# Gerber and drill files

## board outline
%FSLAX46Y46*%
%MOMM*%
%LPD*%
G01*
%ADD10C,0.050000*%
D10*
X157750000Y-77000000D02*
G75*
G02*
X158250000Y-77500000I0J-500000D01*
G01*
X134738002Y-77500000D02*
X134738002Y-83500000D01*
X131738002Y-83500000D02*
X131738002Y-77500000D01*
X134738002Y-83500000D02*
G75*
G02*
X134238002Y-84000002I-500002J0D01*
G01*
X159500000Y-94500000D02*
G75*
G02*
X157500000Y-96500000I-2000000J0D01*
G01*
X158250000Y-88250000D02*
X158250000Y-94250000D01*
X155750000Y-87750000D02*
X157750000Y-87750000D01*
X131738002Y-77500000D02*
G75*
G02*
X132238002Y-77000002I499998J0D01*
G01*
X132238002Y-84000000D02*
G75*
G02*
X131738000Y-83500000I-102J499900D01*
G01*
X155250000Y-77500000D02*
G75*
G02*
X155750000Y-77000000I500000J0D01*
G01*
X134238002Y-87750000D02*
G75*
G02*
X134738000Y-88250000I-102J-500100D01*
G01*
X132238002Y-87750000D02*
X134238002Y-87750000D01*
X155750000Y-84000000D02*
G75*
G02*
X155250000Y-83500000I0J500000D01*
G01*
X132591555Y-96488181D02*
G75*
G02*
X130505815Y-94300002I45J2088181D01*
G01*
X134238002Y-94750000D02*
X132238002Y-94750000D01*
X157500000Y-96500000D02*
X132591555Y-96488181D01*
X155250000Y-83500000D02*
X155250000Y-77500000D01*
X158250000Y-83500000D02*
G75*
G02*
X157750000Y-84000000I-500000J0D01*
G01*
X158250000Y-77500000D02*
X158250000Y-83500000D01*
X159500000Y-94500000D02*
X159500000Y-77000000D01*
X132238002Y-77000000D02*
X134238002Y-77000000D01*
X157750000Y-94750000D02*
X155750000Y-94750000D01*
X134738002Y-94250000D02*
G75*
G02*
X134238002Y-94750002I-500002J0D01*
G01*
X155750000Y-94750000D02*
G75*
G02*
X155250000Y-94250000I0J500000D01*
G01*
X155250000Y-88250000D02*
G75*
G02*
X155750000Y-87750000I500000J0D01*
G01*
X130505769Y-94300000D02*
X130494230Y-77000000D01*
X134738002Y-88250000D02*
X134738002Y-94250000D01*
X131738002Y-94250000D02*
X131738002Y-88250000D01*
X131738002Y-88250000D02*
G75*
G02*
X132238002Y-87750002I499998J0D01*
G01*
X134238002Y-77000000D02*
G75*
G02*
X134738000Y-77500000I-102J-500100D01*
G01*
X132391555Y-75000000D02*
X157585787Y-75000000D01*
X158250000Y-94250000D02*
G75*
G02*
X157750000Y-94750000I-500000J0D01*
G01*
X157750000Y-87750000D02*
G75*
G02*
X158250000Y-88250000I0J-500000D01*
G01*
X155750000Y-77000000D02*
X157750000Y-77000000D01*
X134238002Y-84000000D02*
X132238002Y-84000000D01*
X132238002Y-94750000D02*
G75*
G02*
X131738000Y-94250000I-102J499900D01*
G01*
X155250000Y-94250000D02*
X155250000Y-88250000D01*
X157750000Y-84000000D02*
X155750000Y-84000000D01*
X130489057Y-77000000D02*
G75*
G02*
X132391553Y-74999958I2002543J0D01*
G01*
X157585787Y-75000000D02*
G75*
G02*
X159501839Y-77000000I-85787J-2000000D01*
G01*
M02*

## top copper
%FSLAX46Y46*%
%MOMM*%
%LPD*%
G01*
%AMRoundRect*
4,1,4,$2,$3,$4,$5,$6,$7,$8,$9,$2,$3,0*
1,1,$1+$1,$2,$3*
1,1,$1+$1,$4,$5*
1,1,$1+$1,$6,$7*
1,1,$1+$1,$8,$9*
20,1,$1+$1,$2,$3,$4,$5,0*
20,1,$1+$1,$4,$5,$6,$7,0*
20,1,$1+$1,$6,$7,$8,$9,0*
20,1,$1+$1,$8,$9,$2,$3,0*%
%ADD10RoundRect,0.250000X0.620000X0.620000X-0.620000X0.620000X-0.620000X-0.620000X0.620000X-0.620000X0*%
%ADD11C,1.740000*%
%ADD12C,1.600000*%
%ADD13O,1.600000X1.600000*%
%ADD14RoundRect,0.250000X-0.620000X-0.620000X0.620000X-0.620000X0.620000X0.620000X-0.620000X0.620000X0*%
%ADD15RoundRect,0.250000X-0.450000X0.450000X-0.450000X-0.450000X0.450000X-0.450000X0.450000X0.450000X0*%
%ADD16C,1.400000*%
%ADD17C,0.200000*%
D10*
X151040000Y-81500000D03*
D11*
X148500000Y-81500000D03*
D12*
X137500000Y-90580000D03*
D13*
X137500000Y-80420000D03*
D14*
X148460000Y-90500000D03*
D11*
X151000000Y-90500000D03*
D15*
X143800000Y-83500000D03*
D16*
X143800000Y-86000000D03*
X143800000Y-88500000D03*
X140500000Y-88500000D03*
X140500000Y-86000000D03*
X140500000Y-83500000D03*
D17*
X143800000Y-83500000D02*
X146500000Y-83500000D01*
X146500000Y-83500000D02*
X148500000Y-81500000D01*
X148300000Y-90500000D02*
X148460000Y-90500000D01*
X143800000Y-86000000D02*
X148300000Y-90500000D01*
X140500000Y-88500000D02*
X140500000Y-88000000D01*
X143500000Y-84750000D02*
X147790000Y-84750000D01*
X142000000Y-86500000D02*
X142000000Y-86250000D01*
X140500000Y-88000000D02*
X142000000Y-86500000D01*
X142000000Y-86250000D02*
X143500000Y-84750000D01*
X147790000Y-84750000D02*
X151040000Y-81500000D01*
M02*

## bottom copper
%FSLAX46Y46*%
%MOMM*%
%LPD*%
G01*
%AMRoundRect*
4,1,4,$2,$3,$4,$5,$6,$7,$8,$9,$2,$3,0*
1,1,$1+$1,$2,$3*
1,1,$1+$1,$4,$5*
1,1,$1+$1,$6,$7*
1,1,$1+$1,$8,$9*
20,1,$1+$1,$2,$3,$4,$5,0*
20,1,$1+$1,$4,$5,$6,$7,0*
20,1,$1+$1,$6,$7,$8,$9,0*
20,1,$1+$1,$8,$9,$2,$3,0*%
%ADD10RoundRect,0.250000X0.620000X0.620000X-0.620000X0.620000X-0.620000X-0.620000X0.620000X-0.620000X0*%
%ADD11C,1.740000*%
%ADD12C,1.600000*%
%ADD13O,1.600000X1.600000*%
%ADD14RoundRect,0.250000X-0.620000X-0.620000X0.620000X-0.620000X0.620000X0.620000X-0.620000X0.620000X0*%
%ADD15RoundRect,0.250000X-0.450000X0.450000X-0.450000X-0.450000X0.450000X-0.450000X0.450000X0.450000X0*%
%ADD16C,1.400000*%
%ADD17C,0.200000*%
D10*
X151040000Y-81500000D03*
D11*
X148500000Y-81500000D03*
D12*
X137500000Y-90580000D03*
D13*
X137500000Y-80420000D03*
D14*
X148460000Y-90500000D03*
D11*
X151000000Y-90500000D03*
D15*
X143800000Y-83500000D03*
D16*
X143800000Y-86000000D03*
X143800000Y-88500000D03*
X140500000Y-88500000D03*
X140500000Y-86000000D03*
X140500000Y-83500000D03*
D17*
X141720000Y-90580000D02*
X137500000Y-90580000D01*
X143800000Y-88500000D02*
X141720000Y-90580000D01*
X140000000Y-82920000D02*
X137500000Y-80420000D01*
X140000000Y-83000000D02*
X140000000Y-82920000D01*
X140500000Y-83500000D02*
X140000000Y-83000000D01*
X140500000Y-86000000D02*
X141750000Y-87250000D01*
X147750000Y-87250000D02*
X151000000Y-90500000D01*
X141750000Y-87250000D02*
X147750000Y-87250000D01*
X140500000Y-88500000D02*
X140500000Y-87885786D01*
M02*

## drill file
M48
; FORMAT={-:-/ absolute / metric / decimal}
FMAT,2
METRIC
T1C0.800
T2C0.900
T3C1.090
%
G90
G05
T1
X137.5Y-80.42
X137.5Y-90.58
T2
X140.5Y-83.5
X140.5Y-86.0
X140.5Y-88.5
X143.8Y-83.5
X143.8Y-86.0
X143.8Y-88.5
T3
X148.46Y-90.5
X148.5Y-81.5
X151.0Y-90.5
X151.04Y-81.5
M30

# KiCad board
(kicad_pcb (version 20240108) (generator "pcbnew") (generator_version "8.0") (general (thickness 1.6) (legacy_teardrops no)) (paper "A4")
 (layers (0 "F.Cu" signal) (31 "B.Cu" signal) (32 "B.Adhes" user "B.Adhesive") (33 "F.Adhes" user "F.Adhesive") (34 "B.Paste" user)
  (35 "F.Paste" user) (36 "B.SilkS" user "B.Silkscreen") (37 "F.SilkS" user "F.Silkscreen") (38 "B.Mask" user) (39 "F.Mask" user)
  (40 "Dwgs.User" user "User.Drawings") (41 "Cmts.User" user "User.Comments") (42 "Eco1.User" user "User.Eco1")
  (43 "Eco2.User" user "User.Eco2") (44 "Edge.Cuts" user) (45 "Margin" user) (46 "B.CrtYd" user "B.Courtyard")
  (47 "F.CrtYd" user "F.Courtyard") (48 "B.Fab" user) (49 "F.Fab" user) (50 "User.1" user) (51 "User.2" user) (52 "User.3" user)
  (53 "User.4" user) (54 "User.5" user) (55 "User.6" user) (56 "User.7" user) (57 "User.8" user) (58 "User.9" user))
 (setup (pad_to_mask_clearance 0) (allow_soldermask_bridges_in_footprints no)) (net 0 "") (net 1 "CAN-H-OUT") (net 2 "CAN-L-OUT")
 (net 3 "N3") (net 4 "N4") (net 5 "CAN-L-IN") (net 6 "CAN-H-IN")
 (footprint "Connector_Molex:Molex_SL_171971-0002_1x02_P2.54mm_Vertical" (layer "F.Cu") (at 151.04 81.5 180)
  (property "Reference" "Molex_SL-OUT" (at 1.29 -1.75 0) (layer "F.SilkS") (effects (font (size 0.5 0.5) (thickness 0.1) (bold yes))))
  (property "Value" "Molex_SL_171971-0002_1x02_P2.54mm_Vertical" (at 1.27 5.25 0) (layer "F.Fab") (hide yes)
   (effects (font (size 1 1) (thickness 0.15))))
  (pad "1" thru_hole roundrect (at 0 0 180) (size 1.74 1.74) (drill 1.09) (layers "*.Cu" "*.Mask") (remove_unused_layers no)
   (roundrect_rratio 0.143678) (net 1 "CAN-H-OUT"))
  (pad "2" thru_hole circle (at 2.54 0 180) (size 1.74 1.74) (drill 1.09) (layers "*.Cu" "*.Mask") (remove_unused_layers no)
   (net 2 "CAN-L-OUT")))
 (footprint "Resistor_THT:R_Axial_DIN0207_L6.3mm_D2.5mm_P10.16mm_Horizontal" (layer "F.Cu") (at 137.5 90.58 90)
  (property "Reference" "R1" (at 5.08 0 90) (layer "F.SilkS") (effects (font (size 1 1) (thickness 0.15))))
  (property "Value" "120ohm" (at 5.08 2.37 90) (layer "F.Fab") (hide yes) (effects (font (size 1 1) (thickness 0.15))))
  (pad "1" thru_hole circle (at 0 0 90) (size 1.6 1.6) (drill 0.8) (layers "*.Cu" "*.Mask") (remove_unused_layers no) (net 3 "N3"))
  (pad "2" thru_hole oval (at 10.16 0 90) (size 1.6 1.6) (drill 0.8) (layers "*.Cu" "*.Mask") (remove_unused_layers no) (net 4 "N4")))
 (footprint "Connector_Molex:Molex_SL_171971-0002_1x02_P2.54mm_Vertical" (layer "F.Cu") (at 148.46 90.5)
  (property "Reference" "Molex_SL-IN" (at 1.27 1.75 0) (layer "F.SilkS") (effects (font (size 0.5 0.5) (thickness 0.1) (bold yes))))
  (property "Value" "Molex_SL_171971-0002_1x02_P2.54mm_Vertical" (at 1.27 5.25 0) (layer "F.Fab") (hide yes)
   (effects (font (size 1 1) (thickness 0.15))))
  (pad "1" thru_hole roundrect (at 0 0) (size 1.74 1.74) (drill 1.09) (layers "*.Cu" "*.Mask") (remove_unused_layers no)
   (roundrect_rratio 0.143678) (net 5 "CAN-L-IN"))
  (pad "2" thru_hole circle (at 2.54 0) (size 1.74 1.74) (drill 1.09) (layers "*.Cu" "*.Mask") (remove_unused_layers no) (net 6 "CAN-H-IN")))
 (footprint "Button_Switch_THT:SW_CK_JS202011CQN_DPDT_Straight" (layer "F.Cu") (at 143.8 83.5 -90)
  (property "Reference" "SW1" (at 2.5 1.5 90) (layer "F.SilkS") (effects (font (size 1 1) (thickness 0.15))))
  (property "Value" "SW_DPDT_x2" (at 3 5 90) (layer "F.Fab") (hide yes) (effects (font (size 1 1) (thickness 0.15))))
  (pad "1" thru_hole roundrect (at 0 0 270) (size 1.4 1.4) (drill 0.9) (layers "*.Cu" "*.Mask") (remove_unused_layers no)
   (roundrect_rratio 0.1785714286) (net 2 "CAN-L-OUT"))
  (pad "2" thru_hole circle (at 2.5 0 270) (size 1.4 1.4) (drill 0.9) (layers "*.Cu" "*.Mask") (remove_unused_layers no) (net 5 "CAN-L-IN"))
  (pad "3" thru_hole circle (at 5 0 270) (size 1.4 1.4) (drill 0.9) (layers "*.Cu" "*.Mask") (remove_unused_layers no) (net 3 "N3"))
  (pad "4" thru_hole circle (at 5 3.3 270) (size 1.4 1.4) (drill 0.9) (layers "*.Cu" "*.Mask") (remove_unused_layers no) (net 1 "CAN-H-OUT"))
  (pad "5" thru_hole circle (at 2.5 3.3 270) (size 1.4 1.4) (drill 0.9) (layers "*.Cu" "*.Mask") (remove_unused_layers no)
   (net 6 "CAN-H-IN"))
  (pad "6" thru_hole circle (at 0 3.3 270) (size 1.4 1.4) (drill 0.9) (layers "*.Cu" "*.Mask") (remove_unused_layers no) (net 4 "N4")))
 (gr_arc (start 157.75 77) (mid 158.103553 77.146447) (end 158.25 77.5) (stroke (width 0.05) (type default)) (layer "Edge.Cuts"))
 (gr_line (start 134.738002 77.5) (end 134.738002 83.5) (stroke (width 0.05) (type default)) (layer "Edge.Cuts"))
 (gr_line (start 131.738002 83.5) (end 131.738002 77.5) (stroke (width 0.05) (type default)) (layer "Edge.Cuts"))
 (gr_arc (start 134.738002 83.5) (mid 134.591558 83.85357) (end 134.238002 84) (stroke (width 0.05) (type default)) (layer "Edge.Cuts"))
 (gr_arc (start 159.5 94.5) (mid 158.914214 95.914214) (end 157.5 96.5) (stroke (width 0.05) (type default)) (layer "Edge.Cuts"))
 (gr_line (start 158.25 88.25) (end 158.25 94.25) (stroke (width 0.05) (type default)) (layer "Edge.Cuts"))
 (gr_line (start 155.75 87.75) (end 157.75 87.75) (stroke (width 0.05) (type default)) (layer "Edge.Cuts"))
 (gr_arc (start 131.738002 77.5) (mid 131.884451 77.146463) (end 132.238002 77) (stroke (width 0.05) (type default)) (layer "Edge.Cuts"))
 (gr_arc (start 132.238002 84) (mid 131.884418 83.85357) (end 131.738002 83.5) (stroke (width 0.05) (type default)) (layer "Edge.Cuts"))
 (gr_arc (start 155.25 77.5) (mid 155.396447 77.146447) (end 155.75 77) (stroke (width 0.05) (type default)) (layer "Edge.Cuts"))
 (gr_arc (start 134.238002 87.75) (mid 134.591525 87.896463) (end 134.738002 88.25) (stroke (width 0.05) (type default)) (layer "Edge.Cuts"))
 (gr_line (start 132.238002 87.75) (end 134.238002 87.75) (stroke (width 0.05) (type default)) (layer "Edge.Cuts"))
 (gr_arc (start 155.75 84) (mid 155.396447 83.853553) (end 155.25 83.5) (stroke (width 0.05) (type default)) (layer "Edge.Cuts"))
 (gr_arc (start 132.591555 96.488181) (mid 131.080046 95.840778) (end 130.50577 94.3) (stroke (width 0.05) (type default))
  (layer "Edge.Cuts"))
 (gr_line (start 134.238002 94.75) (end 132.238002 94.75) (stroke (width 0.05) (type default)) (layer "Edge.Cuts"))
 (gr_line (start 157.5 96.5) (end 132.591555 96.488181) (stroke (width 0.05) (type default)) (layer "Edge.Cuts"))
 (gr_line (start 155.25 83.5) (end 155.25 77.5) (stroke (width 0.05) (type default)) (layer "Edge.Cuts"))
 (gr_arc (start 158.25 83.5) (mid 158.103553 83.853553) (end 157.75 84) (stroke (width 0.05) (type default)) (layer "Edge.Cuts"))
 (gr_line (start 158.25 77.5) (end 158.25 83.5) (stroke (width 0.05) (type default)) (layer "Edge.Cuts"))
 (gr_line (start 159.5 94.5) (end 159.5 77) (stroke (width 0.05) (type default)) (layer "Edge.Cuts"))
 (gr_line (start 132.238002 77) (end 134.238002 77) (stroke (width 0.05) (type default)) (layer "Edge.Cuts"))
 (gr_line (start 157.75 94.75) (end 155.75 94.75) (stroke (width 0.05) (type default)) (layer "Edge.Cuts"))
 (gr_arc (start 134.738002 94.25) (mid 134.591558 94.60357) (end 134.238002 94.75) (stroke (width 0.05) (type default)) (layer "Edge.Cuts"))
 (gr_arc (start 155.75 94.75) (mid 155.396447 94.603553) (end 155.25 94.25) (stroke (width 0.05) (type default)) (layer "Edge.Cuts"))
 (gr_arc (start 155.25 88.25) (mid 155.396447 87.896447) (end 155.75 87.75) (stroke (width 0.05) (type default)) (layer "Edge.Cuts"))
 (gr_line (start 130.505769 94.3) (end 130.49423 77) (stroke (width 0.05) (type default)) (layer "Edge.Cuts"))
 (gr_line (start 134.738002 88.25) (end 134.738002 94.25) (stroke (width 0.05) (type default)) (layer "Edge.Cuts"))
 (gr_line (start 131.738002 94.25) (end 131.738002 88.25) (stroke (width 0.05) (type default)) (layer "Edge.Cuts"))
 (gr_arc (start 131.738002 88.25) (mid 131.884451 87.896463) (end 132.238002 87.75) (stroke (width 0.05) (type default)) (layer "Edge.Cuts"))
 (gr_arc (start 134.238002 77) (mid 134.591525 77.146463) (end 134.738002 77.5) (stroke (width 0.05) (type default)) (layer "Edge.Cuts"))
 (gr_line (start 132.391555 75) (end 157.585787 75) (stroke (width 0.05) (type default)) (layer "Edge.Cuts"))
 (gr_arc (start 158.25 94.25) (mid 158.103553 94.603553) (end 157.75 94.75) (stroke (width 0.05) (type default)) (layer "Edge.Cuts"))
 (gr_arc (start 157.75 87.75) (mid 158.103553 87.896447) (end 158.25 88.25) (stroke (width 0.05) (type default)) (layer "Edge.Cuts"))
 (gr_line (start 155.75 77) (end 157.75 77) (stroke (width 0.05) (type default)) (layer "Edge.Cuts"))
 (gr_line (start 134.238002 84) (end 132.238002 84) (stroke (width 0.05) (type default)) (layer "Edge.Cuts"))
 (gr_arc (start 132.238002 94.75) (mid 131.884418 94.60357) (end 131.738002 94.25) (stroke (width 0.05) (type default)) (layer "Edge.Cuts"))
 (gr_line (start 155.25 94.25) (end 155.25 88.25) (stroke (width 0.05) (type default)) (layer "Edge.Cuts"))
 (gr_line (start 157.75 84) (end 155.75 84) (stroke (width 0.05) (type default)) (layer "Edge.Cuts"))
 (gr_arc (start 130.489057 77) (mid 131.04065 75.619828) (end 132.391555 75) (stroke (width 0.05) (type default)) (layer "Edge.Cuts"))
 (gr_arc (start 157.585787 75) (mid 158.945526 75.615148) (end 159.501839 77) (stroke (width 0.05) (type default)) (layer "Edge.Cuts"))
 (segment (start 141.72 90.58) (end 137.5 90.58) (width 0.2) (layer "B.Cu") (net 3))
 (segment (start 143.8 88.5) (end 141.72 90.58) (width 0.2) (layer "B.Cu") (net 3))
 (segment (start 140 82.92) (end 137.5 80.42) (width 0.2) (layer "B.Cu") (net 4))
 (segment (start 140 83) (end 140 82.92) (width 0.2) (layer "B.Cu") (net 4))
 (segment (start 140.5 83.5) (end 140 83) (width 0.2) (layer "B.Cu") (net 4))
 (segment (start 143.8 83.5) (end 146.5 83.5) (width 0.2) (layer "F.Cu") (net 2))
 (segment (start 146.5 83.5) (end 148.5 81.5) (width 0.2) (layer "F.Cu") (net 2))
 (segment (start 148.3 90.5) (end 148.46 90.5) (width 0.2) (layer "F.Cu") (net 5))
 (segment (start 143.8 86) (end 148.3 90.5) (width 0.2) (layer "F.Cu") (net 5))
 (segment (start 140.5 86) (end 141.75 87.25) (width 0.2) (layer "B.Cu") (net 6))
 (segment (start 147.75 87.25) (end 151 90.5) (width 0.2) (layer "B.Cu") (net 6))
 (segment (start 141.75 87.25) (end 147.75 87.25) (width 0.2) (layer "B.Cu") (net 6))
 (segment (start 140.5 88.5) (end 140.5 88) (width 0.2) (layer "F.Cu") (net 1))
 (segment (start 143.5 84.75) (end 147.79 84.75) (width 0.2) (layer "F.Cu") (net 1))
 (segment (start 142 86.5) (end 142 86.25) (width 0.2) (layer "F.Cu") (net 1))
 (segment (start 140.5 88) (end 142 86.5) (width 0.2) (layer "F.Cu") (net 1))
 (segment (start 142 86.25) (end 143.5 84.75) (width 0.2) (layer "F.Cu") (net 1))
 (segment (start 147.79 84.75) (end 151.04 81.5) (width 0.2) (layer "F.Cu") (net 1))
 (segment (start 140.5 88.5) (end 140.5 87.885786) (width 0.2) (layer "B.Cu") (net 1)))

